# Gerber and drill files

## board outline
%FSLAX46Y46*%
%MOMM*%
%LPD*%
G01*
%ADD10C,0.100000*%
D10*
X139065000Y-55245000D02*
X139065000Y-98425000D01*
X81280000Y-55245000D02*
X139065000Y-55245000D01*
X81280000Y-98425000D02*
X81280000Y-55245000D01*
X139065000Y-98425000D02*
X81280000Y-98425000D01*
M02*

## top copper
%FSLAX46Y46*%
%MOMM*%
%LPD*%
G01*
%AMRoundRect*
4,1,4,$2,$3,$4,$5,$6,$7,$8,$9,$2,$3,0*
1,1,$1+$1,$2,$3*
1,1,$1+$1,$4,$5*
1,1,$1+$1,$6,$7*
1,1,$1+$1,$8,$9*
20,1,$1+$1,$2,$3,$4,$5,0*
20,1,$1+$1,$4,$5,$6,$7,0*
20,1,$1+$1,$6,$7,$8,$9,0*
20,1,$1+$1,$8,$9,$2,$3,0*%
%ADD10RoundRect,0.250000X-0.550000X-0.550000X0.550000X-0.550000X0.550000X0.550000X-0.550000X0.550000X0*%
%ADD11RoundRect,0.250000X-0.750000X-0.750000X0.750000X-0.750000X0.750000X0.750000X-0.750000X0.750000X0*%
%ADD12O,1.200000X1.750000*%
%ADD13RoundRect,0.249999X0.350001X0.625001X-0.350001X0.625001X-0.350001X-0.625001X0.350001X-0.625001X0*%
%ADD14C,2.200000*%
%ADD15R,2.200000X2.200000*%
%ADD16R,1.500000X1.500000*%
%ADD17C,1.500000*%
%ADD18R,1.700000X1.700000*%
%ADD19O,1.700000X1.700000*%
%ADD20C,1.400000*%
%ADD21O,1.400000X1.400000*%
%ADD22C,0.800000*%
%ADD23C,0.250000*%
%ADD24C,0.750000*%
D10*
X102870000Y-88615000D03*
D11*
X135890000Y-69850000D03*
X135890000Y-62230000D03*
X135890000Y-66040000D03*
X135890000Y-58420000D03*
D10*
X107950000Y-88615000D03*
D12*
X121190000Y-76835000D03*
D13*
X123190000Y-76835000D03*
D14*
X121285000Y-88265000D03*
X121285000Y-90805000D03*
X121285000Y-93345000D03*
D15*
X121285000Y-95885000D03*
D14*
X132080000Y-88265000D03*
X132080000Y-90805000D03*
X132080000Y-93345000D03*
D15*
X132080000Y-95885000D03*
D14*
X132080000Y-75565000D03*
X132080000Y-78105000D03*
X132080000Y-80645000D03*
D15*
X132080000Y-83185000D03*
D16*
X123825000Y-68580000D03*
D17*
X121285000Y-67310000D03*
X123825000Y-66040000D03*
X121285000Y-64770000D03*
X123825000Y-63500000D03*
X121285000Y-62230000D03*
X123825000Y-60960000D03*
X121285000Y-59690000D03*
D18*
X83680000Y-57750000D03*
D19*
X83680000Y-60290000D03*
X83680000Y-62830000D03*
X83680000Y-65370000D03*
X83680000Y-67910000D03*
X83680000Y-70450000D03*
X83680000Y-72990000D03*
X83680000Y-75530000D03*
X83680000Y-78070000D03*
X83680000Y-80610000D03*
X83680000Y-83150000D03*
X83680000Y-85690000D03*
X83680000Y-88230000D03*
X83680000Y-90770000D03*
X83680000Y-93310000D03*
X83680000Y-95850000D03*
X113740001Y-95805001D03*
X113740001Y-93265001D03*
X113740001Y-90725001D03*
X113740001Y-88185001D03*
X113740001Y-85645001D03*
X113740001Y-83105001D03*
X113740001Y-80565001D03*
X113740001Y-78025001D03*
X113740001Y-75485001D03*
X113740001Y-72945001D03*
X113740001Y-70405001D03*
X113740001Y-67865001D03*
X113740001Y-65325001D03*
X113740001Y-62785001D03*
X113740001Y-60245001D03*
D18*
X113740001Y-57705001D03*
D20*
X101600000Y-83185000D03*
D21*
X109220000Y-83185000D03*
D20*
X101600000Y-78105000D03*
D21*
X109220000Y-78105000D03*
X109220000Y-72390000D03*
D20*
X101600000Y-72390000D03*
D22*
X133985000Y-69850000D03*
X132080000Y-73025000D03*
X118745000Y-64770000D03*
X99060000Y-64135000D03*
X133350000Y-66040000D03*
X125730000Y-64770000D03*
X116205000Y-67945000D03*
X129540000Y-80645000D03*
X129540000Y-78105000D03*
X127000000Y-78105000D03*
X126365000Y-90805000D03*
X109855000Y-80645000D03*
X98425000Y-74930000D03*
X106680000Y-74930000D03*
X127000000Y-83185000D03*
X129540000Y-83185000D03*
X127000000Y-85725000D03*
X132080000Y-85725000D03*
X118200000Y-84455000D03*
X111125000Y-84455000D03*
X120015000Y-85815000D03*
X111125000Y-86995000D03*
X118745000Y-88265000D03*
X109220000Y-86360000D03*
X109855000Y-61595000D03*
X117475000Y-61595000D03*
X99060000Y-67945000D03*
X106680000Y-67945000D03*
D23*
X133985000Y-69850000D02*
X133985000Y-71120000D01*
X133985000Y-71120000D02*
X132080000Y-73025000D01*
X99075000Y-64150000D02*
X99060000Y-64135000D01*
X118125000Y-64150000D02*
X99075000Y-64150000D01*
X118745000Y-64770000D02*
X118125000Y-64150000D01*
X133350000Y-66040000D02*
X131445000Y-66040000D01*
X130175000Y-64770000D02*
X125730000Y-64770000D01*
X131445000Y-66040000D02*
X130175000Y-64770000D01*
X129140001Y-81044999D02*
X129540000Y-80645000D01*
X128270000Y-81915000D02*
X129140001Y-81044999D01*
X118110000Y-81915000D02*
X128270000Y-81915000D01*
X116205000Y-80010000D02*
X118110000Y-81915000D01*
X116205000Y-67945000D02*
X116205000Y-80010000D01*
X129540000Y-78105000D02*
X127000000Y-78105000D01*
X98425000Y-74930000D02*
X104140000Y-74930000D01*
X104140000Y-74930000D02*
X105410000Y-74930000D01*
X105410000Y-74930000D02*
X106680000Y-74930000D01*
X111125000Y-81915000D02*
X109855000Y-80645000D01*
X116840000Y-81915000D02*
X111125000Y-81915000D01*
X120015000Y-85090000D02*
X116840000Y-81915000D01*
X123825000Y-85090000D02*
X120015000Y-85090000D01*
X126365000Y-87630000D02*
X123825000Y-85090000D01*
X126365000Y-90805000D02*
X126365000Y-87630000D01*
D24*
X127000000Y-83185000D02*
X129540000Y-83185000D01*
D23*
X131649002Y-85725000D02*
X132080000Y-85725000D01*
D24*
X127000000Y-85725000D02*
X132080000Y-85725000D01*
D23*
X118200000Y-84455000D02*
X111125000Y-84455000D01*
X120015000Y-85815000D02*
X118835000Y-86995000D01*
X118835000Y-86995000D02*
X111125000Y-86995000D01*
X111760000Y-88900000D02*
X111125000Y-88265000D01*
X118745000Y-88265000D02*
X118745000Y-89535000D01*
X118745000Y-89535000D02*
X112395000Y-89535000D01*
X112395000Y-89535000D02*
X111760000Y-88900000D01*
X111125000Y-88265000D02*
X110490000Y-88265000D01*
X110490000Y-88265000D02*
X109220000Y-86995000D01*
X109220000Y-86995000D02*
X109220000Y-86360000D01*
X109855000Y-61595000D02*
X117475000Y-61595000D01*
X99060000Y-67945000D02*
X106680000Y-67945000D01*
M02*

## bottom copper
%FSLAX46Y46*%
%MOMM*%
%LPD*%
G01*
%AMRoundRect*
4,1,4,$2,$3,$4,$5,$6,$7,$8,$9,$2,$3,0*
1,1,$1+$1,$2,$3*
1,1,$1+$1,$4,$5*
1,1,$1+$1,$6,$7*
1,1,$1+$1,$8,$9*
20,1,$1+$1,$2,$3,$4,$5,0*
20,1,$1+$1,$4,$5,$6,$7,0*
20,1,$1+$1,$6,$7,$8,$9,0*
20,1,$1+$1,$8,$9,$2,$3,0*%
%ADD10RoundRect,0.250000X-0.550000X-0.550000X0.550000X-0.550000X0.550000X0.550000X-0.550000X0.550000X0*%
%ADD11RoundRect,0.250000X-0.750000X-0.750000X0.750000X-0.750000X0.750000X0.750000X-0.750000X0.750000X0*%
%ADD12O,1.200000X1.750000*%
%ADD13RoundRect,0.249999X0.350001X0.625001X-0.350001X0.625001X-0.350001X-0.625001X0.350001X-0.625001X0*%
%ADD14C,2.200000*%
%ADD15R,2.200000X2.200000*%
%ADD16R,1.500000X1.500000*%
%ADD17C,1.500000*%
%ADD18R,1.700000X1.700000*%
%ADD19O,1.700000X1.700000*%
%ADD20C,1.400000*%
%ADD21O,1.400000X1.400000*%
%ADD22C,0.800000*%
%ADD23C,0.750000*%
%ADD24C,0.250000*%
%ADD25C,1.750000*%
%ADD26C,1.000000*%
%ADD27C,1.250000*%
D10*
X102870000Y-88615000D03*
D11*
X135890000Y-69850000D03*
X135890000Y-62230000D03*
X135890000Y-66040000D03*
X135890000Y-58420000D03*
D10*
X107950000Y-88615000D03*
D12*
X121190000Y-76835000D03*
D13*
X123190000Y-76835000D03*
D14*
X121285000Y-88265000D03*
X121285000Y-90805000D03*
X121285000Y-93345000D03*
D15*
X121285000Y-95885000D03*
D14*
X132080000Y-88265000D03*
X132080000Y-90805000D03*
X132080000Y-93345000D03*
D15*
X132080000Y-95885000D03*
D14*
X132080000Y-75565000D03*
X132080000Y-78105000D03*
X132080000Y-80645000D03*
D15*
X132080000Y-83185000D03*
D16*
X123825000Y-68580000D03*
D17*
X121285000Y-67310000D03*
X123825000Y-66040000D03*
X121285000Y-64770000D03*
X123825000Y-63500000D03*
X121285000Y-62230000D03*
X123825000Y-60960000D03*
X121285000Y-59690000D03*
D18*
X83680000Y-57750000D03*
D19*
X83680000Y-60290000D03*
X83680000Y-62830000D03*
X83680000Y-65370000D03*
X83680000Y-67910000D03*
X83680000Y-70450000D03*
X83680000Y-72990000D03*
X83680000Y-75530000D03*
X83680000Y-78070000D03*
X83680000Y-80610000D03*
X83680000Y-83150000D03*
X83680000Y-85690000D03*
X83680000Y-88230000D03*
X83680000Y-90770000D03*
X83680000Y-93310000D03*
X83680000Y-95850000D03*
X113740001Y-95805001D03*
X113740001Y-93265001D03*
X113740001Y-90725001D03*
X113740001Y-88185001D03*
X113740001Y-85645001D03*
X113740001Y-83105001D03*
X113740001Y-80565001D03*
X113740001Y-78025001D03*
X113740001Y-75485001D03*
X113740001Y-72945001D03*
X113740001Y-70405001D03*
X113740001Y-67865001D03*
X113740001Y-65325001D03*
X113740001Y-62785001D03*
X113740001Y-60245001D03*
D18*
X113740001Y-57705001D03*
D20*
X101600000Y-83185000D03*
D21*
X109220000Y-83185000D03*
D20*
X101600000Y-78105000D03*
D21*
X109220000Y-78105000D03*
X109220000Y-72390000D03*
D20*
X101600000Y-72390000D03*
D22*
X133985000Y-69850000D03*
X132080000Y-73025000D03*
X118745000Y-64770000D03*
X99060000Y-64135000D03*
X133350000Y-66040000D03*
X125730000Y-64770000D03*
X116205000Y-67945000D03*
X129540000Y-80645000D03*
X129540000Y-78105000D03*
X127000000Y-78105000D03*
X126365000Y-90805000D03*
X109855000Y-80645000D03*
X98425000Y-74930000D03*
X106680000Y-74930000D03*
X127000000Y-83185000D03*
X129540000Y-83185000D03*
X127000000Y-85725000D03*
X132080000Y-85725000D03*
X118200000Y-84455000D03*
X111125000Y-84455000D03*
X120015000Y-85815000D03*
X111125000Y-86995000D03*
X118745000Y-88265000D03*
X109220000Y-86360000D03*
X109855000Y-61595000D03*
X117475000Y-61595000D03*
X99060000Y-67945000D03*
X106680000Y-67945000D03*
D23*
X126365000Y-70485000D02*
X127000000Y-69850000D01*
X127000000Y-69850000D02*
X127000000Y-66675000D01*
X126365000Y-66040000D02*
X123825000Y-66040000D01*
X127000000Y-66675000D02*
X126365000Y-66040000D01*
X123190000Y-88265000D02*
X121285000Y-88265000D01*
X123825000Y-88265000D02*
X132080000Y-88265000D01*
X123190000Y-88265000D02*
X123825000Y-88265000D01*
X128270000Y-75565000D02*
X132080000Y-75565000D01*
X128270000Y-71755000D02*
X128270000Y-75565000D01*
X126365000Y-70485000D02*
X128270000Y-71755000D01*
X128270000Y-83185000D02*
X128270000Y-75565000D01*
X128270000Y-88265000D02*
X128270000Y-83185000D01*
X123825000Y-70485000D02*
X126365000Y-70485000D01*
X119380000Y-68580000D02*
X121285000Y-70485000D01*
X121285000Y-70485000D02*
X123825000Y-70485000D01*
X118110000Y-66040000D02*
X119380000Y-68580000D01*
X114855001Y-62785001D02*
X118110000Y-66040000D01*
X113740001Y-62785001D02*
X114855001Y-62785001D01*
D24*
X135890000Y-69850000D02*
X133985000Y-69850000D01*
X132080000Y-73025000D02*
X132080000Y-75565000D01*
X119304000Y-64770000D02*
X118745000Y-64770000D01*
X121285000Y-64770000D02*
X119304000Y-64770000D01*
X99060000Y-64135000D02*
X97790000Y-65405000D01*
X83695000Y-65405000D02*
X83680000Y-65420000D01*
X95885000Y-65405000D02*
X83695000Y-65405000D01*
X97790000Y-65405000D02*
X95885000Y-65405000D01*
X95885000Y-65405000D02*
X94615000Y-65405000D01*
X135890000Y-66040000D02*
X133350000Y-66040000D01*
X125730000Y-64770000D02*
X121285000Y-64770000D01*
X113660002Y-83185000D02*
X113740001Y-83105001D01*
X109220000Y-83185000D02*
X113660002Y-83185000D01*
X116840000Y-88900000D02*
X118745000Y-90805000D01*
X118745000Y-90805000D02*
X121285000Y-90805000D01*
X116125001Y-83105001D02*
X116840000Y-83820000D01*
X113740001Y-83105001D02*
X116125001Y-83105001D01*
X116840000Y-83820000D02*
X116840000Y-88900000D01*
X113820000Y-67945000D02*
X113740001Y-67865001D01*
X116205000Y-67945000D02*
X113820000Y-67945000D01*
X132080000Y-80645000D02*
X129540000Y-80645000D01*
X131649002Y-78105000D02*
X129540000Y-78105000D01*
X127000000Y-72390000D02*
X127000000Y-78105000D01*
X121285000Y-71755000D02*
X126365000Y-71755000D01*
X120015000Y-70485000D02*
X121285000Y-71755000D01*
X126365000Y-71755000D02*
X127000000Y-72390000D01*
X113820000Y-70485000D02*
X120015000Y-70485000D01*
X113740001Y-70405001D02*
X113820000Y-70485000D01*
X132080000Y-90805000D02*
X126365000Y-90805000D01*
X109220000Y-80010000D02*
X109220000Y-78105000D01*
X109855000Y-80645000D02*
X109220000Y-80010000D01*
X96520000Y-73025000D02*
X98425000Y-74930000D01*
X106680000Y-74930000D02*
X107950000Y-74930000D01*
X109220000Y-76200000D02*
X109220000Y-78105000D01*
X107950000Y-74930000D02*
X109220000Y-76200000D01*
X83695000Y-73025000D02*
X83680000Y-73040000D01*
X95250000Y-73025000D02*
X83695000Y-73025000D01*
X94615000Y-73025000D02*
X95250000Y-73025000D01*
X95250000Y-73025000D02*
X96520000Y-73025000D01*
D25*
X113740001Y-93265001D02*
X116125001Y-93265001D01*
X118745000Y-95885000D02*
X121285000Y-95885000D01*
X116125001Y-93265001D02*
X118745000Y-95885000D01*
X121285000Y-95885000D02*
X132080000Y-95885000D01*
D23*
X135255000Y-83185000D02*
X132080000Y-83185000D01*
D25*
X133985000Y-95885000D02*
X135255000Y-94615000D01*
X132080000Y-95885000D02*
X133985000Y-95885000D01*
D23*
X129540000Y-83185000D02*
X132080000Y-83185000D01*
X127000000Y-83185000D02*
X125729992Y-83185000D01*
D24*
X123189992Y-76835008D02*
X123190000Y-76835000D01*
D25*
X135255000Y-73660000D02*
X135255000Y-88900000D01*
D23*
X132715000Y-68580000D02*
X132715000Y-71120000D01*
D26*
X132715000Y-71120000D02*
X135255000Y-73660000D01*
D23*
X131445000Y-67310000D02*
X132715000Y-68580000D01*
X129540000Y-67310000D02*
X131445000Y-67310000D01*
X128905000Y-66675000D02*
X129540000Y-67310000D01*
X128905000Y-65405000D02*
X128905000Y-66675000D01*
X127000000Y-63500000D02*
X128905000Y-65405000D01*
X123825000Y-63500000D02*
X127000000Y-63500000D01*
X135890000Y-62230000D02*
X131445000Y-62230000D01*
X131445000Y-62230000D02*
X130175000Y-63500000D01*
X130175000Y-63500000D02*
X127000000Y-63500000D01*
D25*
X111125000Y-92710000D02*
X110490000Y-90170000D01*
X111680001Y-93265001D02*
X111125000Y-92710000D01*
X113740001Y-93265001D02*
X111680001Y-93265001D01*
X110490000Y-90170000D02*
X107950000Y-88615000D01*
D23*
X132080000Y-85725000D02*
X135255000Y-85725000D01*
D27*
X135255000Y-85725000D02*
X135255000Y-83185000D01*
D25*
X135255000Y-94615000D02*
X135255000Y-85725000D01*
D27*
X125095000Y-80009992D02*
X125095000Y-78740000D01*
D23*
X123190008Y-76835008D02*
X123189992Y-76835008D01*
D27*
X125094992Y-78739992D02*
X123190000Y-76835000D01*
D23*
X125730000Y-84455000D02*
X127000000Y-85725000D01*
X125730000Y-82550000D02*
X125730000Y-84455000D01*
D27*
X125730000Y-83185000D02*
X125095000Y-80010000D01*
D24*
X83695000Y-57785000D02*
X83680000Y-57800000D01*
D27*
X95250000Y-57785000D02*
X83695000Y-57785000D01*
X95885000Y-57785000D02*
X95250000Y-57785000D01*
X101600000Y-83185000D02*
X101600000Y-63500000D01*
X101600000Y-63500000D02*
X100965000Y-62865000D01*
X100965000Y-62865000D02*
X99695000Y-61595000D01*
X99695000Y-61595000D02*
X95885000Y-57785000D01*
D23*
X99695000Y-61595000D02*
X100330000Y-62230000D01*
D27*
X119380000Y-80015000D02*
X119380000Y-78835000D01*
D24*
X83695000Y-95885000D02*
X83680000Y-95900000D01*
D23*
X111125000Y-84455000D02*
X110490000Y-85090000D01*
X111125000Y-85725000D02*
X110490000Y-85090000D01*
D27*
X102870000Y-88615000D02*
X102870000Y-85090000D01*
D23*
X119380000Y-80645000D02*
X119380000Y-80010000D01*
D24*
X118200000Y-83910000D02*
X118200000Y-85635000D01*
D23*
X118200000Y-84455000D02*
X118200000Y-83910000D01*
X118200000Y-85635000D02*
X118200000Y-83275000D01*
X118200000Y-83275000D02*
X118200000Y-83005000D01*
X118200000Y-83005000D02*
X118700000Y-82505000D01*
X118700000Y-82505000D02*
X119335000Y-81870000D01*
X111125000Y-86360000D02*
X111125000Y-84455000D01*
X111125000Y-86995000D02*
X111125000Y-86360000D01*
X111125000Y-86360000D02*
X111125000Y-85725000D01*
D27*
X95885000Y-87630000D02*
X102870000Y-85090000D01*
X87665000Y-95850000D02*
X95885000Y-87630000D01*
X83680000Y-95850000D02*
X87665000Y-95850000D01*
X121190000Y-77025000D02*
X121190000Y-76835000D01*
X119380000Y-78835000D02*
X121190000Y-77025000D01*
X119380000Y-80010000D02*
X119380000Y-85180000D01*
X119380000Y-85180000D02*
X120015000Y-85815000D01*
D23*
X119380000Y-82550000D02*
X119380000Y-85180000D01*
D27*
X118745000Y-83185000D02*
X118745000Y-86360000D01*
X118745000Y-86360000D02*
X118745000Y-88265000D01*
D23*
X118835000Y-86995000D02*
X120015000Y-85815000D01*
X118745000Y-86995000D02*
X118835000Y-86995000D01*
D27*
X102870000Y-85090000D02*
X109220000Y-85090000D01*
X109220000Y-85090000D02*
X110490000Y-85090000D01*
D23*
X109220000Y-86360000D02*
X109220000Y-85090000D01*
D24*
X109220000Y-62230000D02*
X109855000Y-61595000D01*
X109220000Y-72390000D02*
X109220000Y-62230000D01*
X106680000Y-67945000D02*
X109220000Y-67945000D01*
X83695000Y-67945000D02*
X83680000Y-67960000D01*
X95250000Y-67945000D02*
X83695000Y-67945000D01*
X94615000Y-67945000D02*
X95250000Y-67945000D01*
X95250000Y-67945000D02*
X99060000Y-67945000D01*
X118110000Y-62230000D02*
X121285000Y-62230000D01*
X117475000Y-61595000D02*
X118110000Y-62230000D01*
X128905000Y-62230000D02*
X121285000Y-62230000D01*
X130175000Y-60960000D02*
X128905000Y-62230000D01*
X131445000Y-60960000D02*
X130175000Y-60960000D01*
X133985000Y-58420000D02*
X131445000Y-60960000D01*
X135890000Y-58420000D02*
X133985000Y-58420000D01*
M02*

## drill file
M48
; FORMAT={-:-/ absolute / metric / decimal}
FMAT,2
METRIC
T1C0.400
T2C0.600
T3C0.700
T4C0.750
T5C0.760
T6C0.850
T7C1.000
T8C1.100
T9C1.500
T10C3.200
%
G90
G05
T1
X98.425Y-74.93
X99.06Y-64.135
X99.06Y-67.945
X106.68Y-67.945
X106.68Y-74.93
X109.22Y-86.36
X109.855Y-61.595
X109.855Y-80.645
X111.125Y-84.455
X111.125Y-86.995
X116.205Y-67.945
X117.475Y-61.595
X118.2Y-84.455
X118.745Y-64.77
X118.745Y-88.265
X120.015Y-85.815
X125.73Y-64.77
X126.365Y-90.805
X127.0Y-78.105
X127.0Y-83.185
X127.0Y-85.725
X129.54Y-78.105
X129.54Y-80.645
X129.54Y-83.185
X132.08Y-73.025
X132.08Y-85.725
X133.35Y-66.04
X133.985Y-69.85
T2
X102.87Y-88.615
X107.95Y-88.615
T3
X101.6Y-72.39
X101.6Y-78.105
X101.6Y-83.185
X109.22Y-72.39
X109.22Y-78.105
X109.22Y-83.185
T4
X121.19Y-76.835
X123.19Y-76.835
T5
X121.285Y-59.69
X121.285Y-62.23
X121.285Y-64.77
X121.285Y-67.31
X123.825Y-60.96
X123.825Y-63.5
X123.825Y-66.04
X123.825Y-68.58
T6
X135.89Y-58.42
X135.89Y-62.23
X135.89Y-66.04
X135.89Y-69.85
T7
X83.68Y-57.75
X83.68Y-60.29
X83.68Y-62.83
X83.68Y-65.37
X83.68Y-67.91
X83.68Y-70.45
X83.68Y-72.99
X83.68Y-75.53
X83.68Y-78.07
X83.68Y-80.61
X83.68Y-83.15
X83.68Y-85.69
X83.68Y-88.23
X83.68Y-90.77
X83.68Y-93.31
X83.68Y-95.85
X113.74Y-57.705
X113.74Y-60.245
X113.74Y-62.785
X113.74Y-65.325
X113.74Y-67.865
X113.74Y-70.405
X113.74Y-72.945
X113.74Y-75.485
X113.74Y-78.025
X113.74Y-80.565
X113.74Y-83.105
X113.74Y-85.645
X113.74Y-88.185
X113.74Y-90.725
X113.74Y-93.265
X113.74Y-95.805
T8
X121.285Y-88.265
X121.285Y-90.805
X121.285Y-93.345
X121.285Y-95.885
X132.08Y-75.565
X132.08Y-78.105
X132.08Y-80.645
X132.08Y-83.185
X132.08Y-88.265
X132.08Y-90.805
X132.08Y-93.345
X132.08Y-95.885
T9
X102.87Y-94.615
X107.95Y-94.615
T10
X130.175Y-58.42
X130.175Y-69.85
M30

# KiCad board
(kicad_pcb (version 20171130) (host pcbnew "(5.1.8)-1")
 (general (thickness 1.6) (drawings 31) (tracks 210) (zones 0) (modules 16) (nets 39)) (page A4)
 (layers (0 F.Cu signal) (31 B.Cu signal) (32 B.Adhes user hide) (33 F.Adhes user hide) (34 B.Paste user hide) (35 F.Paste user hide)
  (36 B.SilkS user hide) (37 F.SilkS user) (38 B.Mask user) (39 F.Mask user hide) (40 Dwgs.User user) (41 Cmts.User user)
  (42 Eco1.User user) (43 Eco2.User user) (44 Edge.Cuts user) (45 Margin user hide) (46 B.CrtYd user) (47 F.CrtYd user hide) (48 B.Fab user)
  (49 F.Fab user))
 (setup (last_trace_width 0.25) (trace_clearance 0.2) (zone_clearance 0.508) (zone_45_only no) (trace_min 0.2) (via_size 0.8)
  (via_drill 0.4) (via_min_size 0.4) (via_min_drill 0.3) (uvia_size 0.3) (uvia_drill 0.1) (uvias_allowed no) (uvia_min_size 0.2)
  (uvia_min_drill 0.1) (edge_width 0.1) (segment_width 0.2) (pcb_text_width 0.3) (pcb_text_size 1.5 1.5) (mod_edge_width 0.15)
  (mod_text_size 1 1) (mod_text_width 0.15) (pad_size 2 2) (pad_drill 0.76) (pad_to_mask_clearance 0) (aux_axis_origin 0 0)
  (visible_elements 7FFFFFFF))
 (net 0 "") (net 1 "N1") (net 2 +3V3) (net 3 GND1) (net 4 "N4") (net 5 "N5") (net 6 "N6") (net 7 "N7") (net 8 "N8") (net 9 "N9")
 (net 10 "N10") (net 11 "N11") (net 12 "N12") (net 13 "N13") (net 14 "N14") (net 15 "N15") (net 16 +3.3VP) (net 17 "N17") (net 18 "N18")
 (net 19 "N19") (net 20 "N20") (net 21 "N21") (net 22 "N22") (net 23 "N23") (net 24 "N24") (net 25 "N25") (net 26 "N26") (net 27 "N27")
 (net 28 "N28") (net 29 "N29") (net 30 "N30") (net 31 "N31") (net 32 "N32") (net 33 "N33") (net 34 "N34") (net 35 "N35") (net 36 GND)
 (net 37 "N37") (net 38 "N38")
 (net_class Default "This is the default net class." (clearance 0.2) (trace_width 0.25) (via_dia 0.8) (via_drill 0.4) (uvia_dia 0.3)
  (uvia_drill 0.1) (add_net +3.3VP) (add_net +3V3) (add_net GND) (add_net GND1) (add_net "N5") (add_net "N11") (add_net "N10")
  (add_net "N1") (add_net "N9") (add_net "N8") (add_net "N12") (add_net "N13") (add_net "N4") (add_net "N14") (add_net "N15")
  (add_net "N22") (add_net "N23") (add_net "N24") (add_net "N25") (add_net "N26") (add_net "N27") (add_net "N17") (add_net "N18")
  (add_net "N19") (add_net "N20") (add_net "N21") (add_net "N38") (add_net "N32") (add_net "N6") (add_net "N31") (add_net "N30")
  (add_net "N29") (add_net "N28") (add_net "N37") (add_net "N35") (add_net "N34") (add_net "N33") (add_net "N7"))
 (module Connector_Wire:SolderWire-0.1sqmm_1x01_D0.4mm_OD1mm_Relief (layer F.Cu) (at 102.87 88.615)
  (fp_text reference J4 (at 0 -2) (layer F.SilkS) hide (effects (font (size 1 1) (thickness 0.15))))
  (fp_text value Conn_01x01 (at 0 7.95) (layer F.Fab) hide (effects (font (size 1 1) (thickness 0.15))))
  (pad "" np_thru_hole circle (at 0 6) (size 1.5 1.5) (drill 1.5) (layers *.Cu *.Mask))
  (pad 1 thru_hole roundrect (at 0 0) (size 1.6 1.6) (drill 0.6) (layers *.Cu *.Mask) (roundrect_rratio 0.15625) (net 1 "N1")))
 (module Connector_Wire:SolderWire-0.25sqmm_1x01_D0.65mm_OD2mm (layer F.Cu) (at 135.89 69.85)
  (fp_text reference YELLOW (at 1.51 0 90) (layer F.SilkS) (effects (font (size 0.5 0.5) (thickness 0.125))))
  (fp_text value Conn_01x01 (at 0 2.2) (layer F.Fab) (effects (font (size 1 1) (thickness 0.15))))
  (pad 1 thru_hole roundrect (at 0 0) (size 2 2) (drill 0.85) (layers *.Cu *.Mask) (roundrect_rratio 0.125) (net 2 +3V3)))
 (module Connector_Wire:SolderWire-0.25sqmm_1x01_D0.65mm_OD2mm (layer F.Cu) (at 135.89 62.23)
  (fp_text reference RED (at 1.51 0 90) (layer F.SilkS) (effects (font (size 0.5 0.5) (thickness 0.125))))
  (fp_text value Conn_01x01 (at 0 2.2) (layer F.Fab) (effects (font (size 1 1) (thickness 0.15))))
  (pad 1 thru_hole roundrect (at 0 0) (size 2 2) (drill 0.85) (layers *.Cu *.Mask) (roundrect_rratio 0.125) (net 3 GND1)))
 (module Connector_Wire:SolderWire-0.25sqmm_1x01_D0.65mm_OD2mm (layer F.Cu) (at 135.89 66.04)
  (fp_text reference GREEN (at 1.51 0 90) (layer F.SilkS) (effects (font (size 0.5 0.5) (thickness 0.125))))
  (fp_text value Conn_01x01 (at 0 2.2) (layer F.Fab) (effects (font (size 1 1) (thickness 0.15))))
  (pad 1 thru_hole roundrect (at 0 0) (size 2 2) (drill 0.85) (layers *.Cu *.Mask) (roundrect_rratio 0.125) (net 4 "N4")))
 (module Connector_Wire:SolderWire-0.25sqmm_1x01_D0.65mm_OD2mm (layer F.Cu) (at 135.89 58.42)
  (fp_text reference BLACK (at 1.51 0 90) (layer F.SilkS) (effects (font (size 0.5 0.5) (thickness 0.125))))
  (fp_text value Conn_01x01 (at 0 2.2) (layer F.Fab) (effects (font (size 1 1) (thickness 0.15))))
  (pad 1 thru_hole roundrect (at 0 0) (size 2 2) (drill 0.85) (layers *.Cu *.Mask) (roundrect_rratio 0.125) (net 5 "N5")))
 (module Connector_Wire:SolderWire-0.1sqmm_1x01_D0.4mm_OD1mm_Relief (layer F.Cu) (at 107.95 88.615)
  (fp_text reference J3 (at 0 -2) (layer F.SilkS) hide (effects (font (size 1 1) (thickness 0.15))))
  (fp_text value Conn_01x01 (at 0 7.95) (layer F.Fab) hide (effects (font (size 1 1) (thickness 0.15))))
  (pad "" np_thru_hole circle (at 0 6) (size 1.5 1.5) (drill 1.5) (layers *.Cu *.Mask))
  (pad 1 thru_hole roundrect (at 0 0) (size 1.6 1.6) (drill 0.6) (layers *.Cu *.Mask) (roundrect_rratio 0.15625) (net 3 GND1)))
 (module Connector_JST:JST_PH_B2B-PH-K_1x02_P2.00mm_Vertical (layer F.Cu) (at 123.19 76.835 180)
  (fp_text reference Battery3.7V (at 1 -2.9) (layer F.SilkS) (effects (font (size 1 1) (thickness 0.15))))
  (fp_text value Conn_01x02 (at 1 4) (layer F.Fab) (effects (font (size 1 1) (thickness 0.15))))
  (pad 2 thru_hole oval (at 2 0 180) (size 1.2 1.75) (drill 0.75) (layers *.Cu *.Mask) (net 1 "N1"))
  (pad 1 thru_hole roundrect (at 0 0 180) (size 1.2 1.75) (drill 0.75) (layers *.Cu *.Mask) (roundrect_rratio 0.2083325) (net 3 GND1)))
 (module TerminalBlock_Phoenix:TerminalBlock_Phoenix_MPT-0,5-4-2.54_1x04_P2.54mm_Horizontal (layer F.Cu) (at 121.285 95.885 90)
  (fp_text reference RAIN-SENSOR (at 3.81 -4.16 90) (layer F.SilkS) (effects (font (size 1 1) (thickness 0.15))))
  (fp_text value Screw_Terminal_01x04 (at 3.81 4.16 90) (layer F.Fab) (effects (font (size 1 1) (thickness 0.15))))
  (pad 4 thru_hole circle (at 7.62 0 90) (size 2.2 2.2) (drill 1.1) (layers *.Cu *.Mask) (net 2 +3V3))
  (pad 3 thru_hole circle (at 5.08 0 90) (size 2.2 2.2) (drill 1.1) (layers *.Cu *.Mask) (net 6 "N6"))
  (pad 2 thru_hole circle (at 2.54 0 90) (size 2.2 2.2) (drill 1.1) (layers *.Cu *.Mask) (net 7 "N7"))
  (pad 1 thru_hole rect (at 0 0 90) (size 2.2 2.2) (drill 1.1) (layers *.Cu *.Mask) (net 3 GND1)))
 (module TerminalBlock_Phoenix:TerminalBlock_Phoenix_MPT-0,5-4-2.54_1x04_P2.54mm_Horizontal (layer F.Cu) (at 132.08 95.885 90)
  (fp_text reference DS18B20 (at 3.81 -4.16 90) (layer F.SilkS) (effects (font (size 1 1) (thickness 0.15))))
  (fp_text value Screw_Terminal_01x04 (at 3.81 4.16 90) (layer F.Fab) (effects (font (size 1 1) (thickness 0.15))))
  (pad 4 thru_hole circle (at 7.62 0 90) (size 2.2 2.2) (drill 1.1) (layers *.Cu *.Mask) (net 2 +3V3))
  (pad 3 thru_hole circle (at 5.08 0 90) (size 2.2 2.2) (drill 1.1) (layers *.Cu *.Mask) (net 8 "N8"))
  (pad 2 thru_hole circle (at 2.54 0 90) (size 2.2 2.2) (drill 1.1) (layers *.Cu *.Mask) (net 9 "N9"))
  (pad 1 thru_hole rect (at 0 0 90) (size 2.2 2.2) (drill 1.1) (layers *.Cu *.Mask) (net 3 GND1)))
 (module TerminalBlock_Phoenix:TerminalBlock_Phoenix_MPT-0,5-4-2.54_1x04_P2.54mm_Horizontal (layer F.Cu) (at 132.08 83.185 90)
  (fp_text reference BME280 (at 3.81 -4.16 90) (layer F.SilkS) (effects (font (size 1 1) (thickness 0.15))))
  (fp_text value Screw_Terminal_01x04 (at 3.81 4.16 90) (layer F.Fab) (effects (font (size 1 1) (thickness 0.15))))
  (pad 4 thru_hole circle (at 7.62 0 90) (size 2.2 2.2) (drill 1.1) (layers *.Cu *.Mask) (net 2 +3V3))
  (pad 3 thru_hole circle (at 5.08 0 90) (size 2.2 2.2) (drill 1.1) (layers *.Cu *.Mask) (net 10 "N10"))
  (pad 2 thru_hole circle (at 2.54 0 90) (size 2.2 2.2) (drill 1.1) (layers *.Cu *.Mask) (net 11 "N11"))
  (pad 1 thru_hole rect (at 0 0 90) (size 2.2 2.2) (drill 1.1) (layers *.Cu *.Mask) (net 3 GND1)))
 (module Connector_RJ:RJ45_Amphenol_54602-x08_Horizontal (layer F.Cu) (at 123.825 68.58 90)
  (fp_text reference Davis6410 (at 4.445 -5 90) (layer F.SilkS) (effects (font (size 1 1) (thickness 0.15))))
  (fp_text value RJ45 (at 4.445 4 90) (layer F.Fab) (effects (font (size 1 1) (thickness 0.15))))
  (pad "" np_thru_hole circle (at 10.16 6.35 90) (size 3.2 3.2) (drill 3.2) (layers *.Cu *.Mask))
  (pad "" np_thru_hole circle (at -1.27 6.35 90) (size 3.2 3.2) (drill 3.2) (layers *.Cu *.Mask))
  (pad 1 thru_hole rect (at 0 0 90) (size 1.5 1.5) (drill 0.76) (layers *.Cu *.Mask) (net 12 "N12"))
  (pad 2 thru_hole circle (at 1.27 -2.54 90) (size 1.5 1.5) (drill 0.76) (layers *.Cu *.Mask) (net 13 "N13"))
  (pad 3 thru_hole circle (at 2.54 0 90) (size 1.5 1.5) (drill 0.76) (layers *.Cu *.Mask) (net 2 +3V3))
  (pad 4 thru_hole circle (at 3.81 -2.54 90) (size 1.5 1.5) (drill 0.76) (layers *.Cu *.Mask) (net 4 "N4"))
  (pad 5 thru_hole circle (at 5.08 0 90) (size 1.5 1.5) (drill 0.76) (layers *.Cu *.Mask) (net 3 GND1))
  (pad 6 thru_hole circle (at 6.35 -2.54 90) (size 1.5 1.5) (drill 0.76) (layers *.Cu *.Mask) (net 5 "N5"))
  (pad 7 thru_hole circle (at 7.62 0 90) (size 1.5 1.5) (drill 0.76) (layers *.Cu *.Mask) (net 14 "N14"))
  (pad 8 thru_hole circle (at 8.89 -2.54 90) (size 1.5 1.5) (drill 0.76) (layers *.Cu *.Mask) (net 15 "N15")))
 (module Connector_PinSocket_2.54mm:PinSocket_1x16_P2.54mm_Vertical (layer F.Cu) (at 83.68 57.75)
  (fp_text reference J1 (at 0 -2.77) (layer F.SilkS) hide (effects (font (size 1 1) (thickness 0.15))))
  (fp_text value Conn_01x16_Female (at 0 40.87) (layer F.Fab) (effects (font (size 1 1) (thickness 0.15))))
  (pad 1 thru_hole rect (at 0 0) (size 1.7 1.7) (drill 1) (layers *.Cu *.Mask) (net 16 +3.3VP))
  (pad 2 thru_hole oval (at 0 2.54) (size 1.7 1.7) (drill 1) (layers *.Cu *.Mask) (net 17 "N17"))
  (pad 3 thru_hole oval (at 0 5.08) (size 1.7 1.7) (drill 1) (layers *.Cu *.Mask) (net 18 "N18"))
  (pad 4 thru_hole oval (at 0 7.62) (size 1.7 1.7) (drill 1) (layers *.Cu *.Mask) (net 4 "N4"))
  (pad 5 thru_hole oval (at 0 10.16) (size 1.7 1.7) (drill 1) (layers *.Cu *.Mask) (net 5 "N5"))
  (pad 6 thru_hole oval (at 0 12.7) (size 1.7 1.7) (drill 1) (layers *.Cu *.Mask) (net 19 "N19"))
  (pad 7 thru_hole oval (at 0 15.24) (size 1.7 1.7) (drill 1) (layers *.Cu *.Mask) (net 8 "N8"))
  (pad 8 thru_hole oval (at 0 17.78) (size 1.7 1.7) (drill 1) (layers *.Cu *.Mask) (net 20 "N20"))
  (pad 9 thru_hole oval (at 0 20.32) (size 1.7 1.7) (drill 1) (layers *.Cu *.Mask) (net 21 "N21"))
  (pad 10 thru_hole oval (at 0 22.86) (size 1.7 1.7) (drill 1) (layers *.Cu *.Mask) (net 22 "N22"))
  (pad 11 thru_hole oval (at 0 25.4) (size 1.7 1.7) (drill 1) (layers *.Cu *.Mask) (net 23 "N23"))
  (pad 12 thru_hole oval (at 0 27.94) (size 1.7 1.7) (drill 1) (layers *.Cu *.Mask) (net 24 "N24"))
  (pad 13 thru_hole oval (at 0 30.48) (size 1.7 1.7) (drill 1) (layers *.Cu *.Mask) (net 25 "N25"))
  (pad 14 thru_hole oval (at 0 33.02) (size 1.7 1.7) (drill 1) (layers *.Cu *.Mask) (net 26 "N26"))
  (pad 15 thru_hole oval (at 0 35.56) (size 1.7 1.7) (drill 1) (layers *.Cu *.Mask) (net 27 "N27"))
  (pad 16 thru_hole oval (at 0 38.1) (size 1.7 1.7) (drill 1) (layers *.Cu *.Mask) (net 1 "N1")))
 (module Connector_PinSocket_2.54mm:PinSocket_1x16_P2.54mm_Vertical (layer F.Cu) (at 113.740001 57.705001)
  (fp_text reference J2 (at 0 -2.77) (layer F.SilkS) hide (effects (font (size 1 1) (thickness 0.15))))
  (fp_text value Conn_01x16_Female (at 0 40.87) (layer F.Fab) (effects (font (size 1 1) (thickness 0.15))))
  (pad 16 thru_hole oval (at 0 38.1) (size 1.7 1.7) (drill 1) (layers *.Cu *.Mask) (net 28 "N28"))
  (pad 15 thru_hole oval (at 0 35.56) (size 1.7 1.7) (drill 1) (layers *.Cu *.Mask) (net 3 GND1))
  (pad 14 thru_hole oval (at 0 33.02) (size 1.7 1.7) (drill 1) (layers *.Cu *.Mask) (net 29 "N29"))
  (pad 13 thru_hole oval (at 0 30.48) (size 1.7 1.7) (drill 1) (layers *.Cu *.Mask) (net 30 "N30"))
  (pad 12 thru_hole oval (at 0 27.94) (size 1.7 1.7) (drill 1) (layers *.Cu *.Mask) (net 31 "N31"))
  (pad 11 thru_hole oval (at 0 25.4) (size 1.7 1.7) (drill 1) (layers *.Cu *.Mask) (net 6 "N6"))
  (pad 10 thru_hole oval (at 0 22.86) (size 1.7 1.7) (drill 1) (layers *.Cu *.Mask) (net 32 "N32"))
  (pad 9 thru_hole oval (at 0 20.32) (size 1.7 1.7) (drill 1) (layers *.Cu *.Mask) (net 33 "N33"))
  (pad 8 thru_hole oval (at 0 17.78) (size 1.7 1.7) (drill 1) (layers *.Cu *.Mask) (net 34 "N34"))
  (pad 7 thru_hole oval (at 0 15.24) (size 1.7 1.7) (drill 1) (layers *.Cu *.Mask) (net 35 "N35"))
  (pad 6 thru_hole oval (at 0 12.7) (size 1.7 1.7) (drill 1) (layers *.Cu *.Mask) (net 10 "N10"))
  (pad 5 thru_hole oval (at 0 10.16) (size 1.7 1.7) (drill 1) (layers *.Cu *.Mask) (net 11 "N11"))
  (pad 4 thru_hole oval (at 0 7.62) (size 1.7 1.7) (drill 1) (layers *.Cu *.Mask) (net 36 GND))
  (pad 3 thru_hole oval (at 0 5.08) (size 1.7 1.7) (drill 1) (layers *.Cu *.Mask) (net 2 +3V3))
  (pad 2 thru_hole oval (at 0 2.54) (size 1.7 1.7) (drill 1) (layers *.Cu *.Mask) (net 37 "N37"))
  (pad 1 thru_hole rect (at 0 0) (size 1.7 1.7) (drill 1) (layers *.Cu *.Mask) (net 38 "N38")))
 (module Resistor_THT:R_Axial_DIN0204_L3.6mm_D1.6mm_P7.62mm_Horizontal (layer F.Cu) (at 101.6 83.185)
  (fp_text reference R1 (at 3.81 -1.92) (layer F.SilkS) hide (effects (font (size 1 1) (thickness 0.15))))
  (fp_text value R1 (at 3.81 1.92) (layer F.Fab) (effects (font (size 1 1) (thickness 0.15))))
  (pad 1 thru_hole circle (at 0 0) (size 1.4 1.4) (drill 0.7) (layers *.Cu *.Mask) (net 16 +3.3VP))
  (pad 2 thru_hole oval (at 7.62 0) (size 1.4 1.4) (drill 0.7) (layers *.Cu *.Mask) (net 6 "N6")))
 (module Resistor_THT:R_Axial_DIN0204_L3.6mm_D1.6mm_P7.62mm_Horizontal (layer F.Cu) (at 101.6 78.105)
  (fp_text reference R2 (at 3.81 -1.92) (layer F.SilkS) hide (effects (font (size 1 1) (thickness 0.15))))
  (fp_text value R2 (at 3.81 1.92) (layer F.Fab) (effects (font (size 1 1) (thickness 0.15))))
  (pad 1 thru_hole circle (at 0 0) (size 1.4 1.4) (drill 0.7) (layers *.Cu *.Mask) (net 16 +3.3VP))
  (pad 2 thru_hole oval (at 7.62 0) (size 1.4 1.4) (drill 0.7) (layers *.Cu *.Mask) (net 8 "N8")))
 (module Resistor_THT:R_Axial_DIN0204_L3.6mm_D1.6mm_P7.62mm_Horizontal (layer F.Cu) (at 101.6 72.39)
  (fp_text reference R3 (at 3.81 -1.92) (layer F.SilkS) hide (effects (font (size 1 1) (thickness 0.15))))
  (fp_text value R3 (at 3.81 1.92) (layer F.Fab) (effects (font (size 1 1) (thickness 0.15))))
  (pad 2 thru_hole oval (at 7.62 0) (size 1.4 1.4) (drill 0.7) (layers *.Cu *.Mask) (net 5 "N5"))
  (pad 1 thru_hole circle (at 0 0) (size 1.4 1.4) (drill 0.7) (layers *.Cu *.Mask) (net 16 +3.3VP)))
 (gr_line (start 139.065 55.245) (end 139.065 98.425) (layer Edge.Cuts) (width 0.1))
 (gr_line (start 81.28 55.245) (end 139.065 55.245) (layer Edge.Cuts) (width 0.1))
 (gr_line (start 81.28 98.425) (end 81.28 55.245) (layer Edge.Cuts) (width 0.1))
 (gr_line (start 139.065 98.425) (end 81.28 98.425) (layer Edge.Cuts) (width 0.1))
 (segment (start 126.365 70.485) (end 127 69.85) (width 0.75) (layer B.Cu) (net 2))
 (segment (start 127 69.85) (end 127 66.675) (width 0.75) (layer B.Cu) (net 2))
 (segment (start 126.365 66.04) (end 123.825 66.04) (width 0.75) (layer B.Cu) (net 2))
 (segment (start 127 66.675) (end 126.365 66.04) (width 0.75) (layer B.Cu) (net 2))
 (segment (start 123.19 88.265) (end 121.285 88.265) (width 0.75) (layer B.Cu) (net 2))
 (segment (start 123.825 88.265) (end 132.08 88.265) (width 0.75) (layer B.Cu) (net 2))
 (segment (start 123.19 88.265) (end 123.825 88.265) (width 0.75) (layer B.Cu) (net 2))
 (segment (start 128.27 75.565) (end 132.08 75.565) (width 0.75) (layer B.Cu) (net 2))
 (segment (start 128.27 71.755) (end 128.27 75.565) (width 0.75) (layer B.Cu) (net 2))
 (segment (start 126.365 70.485) (end 128.27 71.755) (width 0.75) (layer B.Cu) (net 2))
 (segment (start 128.27 83.185) (end 128.27 75.565) (width 0.75) (layer B.Cu) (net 2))
 (segment (start 128.27 88.265) (end 128.27 83.185) (width 0.75) (layer B.Cu) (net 2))
 (segment (start 123.825 70.485) (end 126.365 70.485) (width 0.75) (layer B.Cu) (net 2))
 (segment (start 119.38 68.58) (end 121.285 70.485) (width 0.75) (layer B.Cu) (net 2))
 (segment (start 121.285 70.485) (end 123.825 70.485) (width 0.75) (layer B.Cu) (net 2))
 (segment (start 118.11 66.04) (end 119.38 68.58) (width 0.75) (layer B.Cu) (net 2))
 (segment (start 114.855001 62.785001) (end 118.11 66.04) (width 0.75) (layer B.Cu) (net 2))
 (segment (start 113.740001 62.785001) (end 114.855001 62.785001) (width 0.75) (layer B.Cu) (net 2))
 (via (at 133.985 69.85) (size 0.8) (drill 0.4) (layers F.Cu B.Cu) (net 2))
 (segment (start 135.89 69.85) (end 133.985 69.85) (width 0.25) (layer B.Cu) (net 2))
 (segment (start 133.985 69.85) (end 133.985 71.12) (width 0.25) (layer F.Cu) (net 2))
 (via (at 132.08 73.025) (size 0.8) (drill 0.4) (layers F.Cu B.Cu) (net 2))
 (segment (start 133.985 71.12) (end 132.08 73.025) (width 0.25) (layer F.Cu) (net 2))
 (segment (start 132.08 73.025) (end 132.08 75.565) (width 0.25) (layer B.Cu) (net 2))
 (via (at 118.745 64.77) (size 0.8) (drill 0.4) (layers F.Cu B.Cu) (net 4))
 (segment (start 119.304 64.77) (end 118.745 64.77) (width 0.25) (layer B.Cu) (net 4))
 (segment (start 121.285 64.77) (end 119.304 64.77) (width 0.25) (layer B.Cu) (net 4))
 (via (at 99.06 64.135) (size 0.8) (drill 0.4) (layers F.Cu B.Cu) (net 4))
 (segment (start 99.075 64.15) (end 99.06 64.135) (width 0.25) (layer F.Cu) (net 4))
 (segment (start 118.125 64.15) (end 99.075 64.15) (width 0.25) (layer F.Cu) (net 4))
 (segment (start 118.745 64.77) (end 118.125 64.15) (width 0.25) (layer F.Cu) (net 4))
 (segment (start 99.06 64.135) (end 97.79 65.405) (width 0.25) (layer B.Cu) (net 4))
 (segment (start 83.695 65.405) (end 83.68 65.42) (width 0.25) (layer B.Cu) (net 4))
 (segment (start 95.885 65.405) (end 83.695 65.405) (width 0.25) (layer B.Cu) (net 4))
 (segment (start 97.79 65.405) (end 95.885 65.405) (width 0.25) (layer B.Cu) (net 4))
 (segment (start 95.885 65.405) (end 94.615 65.405) (width 0.25) (layer B.Cu) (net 4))
 (via (at 133.35 66.04) (size 0.8) (drill 0.4) (layers F.Cu B.Cu) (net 4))
 (segment (start 135.89 66.04) (end 133.35 66.04) (width 0.25) (layer B.Cu) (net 4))
 (segment (start 133.35 66.04) (end 131.445 66.04) (width 0.25) (layer F.Cu) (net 4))
 (via (at 125.73 64.77) (size 0.8) (drill 0.4) (layers F.Cu B.Cu) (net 4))
 (segment (start 130.175 64.77) (end 125.73 64.77) (width 0.25) (layer F.Cu) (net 4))
 (segment (start 131.445 66.04) (end 130.175 64.77) (width 0.25) (layer F.Cu) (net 4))
 (segment (start 125.73 64.77) (end 121.285 64.77) (width 0.25) (layer B.Cu) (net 4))
 (segment (start 113.660002 83.185) (end 113.740001 83.105001) (width 0.25) (layer B.Cu) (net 6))
 (segment (start 109.22 83.185) (end 113.660002 83.185) (width 0.25) (layer B.Cu) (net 6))
 (segment (start 116.84 88.9) (end 118.745 90.805) (width 0.25) (layer B.Cu) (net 6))
 (segment (start 118.745 90.805) (end 121.285 90.805) (width 0.25) (layer B.Cu) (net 6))
 (segment (start 116.125001 83.105001) (end 116.84 83.82) (width 0.25) (layer B.Cu) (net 6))
 (segment (start 113.740001 83.105001) (end 116.125001 83.105001) (width 0.25) (layer B.Cu) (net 6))
 (segment (start 116.84 83.82) (end 116.84 88.9) (width 0.25) (layer B.Cu) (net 6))
 (via (at 116.205 67.945) (size 0.8) (drill 0.4) (layers F.Cu B.Cu) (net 11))
 (segment (start 113.82 67.945) (end 113.740001 67.865001) (width 0.25) (layer B.Cu) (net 11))
 (segment (start 116.205 67.945) (end 113.82 67.945) (width 0.25) (layer B.Cu) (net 11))
 (segment (start 132.08 80.645) (end 129.54 80.645) (width 0.25) (layer B.Cu) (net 11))
 (via (at 129.54 80.645) (size 0.8) (drill 0.4) (layers F.Cu B.Cu) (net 11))
 (segment (start 129.140001 81.044999) (end 129.54 80.645) (width 0.25) (layer F.Cu) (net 11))
 (segment (start 128.27 81.915) (end 129.140001 81.044999) (width 0.25) (layer F.Cu) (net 11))
 (segment (start 118.11 81.915) (end 128.27 81.915) (width 0.25) (layer F.Cu) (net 11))
 (segment (start 116.205 80.01) (end 118.11 81.915) (width 0.25) (layer F.Cu) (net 11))
 (segment (start 116.205 67.945) (end 116.205 80.01) (width 0.25) (layer F.Cu) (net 11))
 (segment (start 131.649002 78.105) (end 129.54 78.105) (width 0.25) (layer B.Cu) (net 10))
 (via (at 129.54 78.105) (size 0.8) (drill 0.4) (layers F.Cu B.Cu) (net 10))
 (segment (start 129.54 78.105) (end 127 78.105) (width 0.25) (layer F.Cu) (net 10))
 (via (at 127 78.105) (size 0.8) (drill 0.4) (layers F.Cu B.Cu) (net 10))
 (segment (start 127 72.39) (end 127 78.105) (width 0.25) (layer B.Cu) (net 10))
 (segment (start 121.285 71.755) (end 126.365 71.755) (width 0.25) (layer B.Cu) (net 10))
 (segment (start 120.015 70.485) (end 121.285 71.755) (width 0.25) (layer B.Cu) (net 10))
 (segment (start 126.365 71.755) (end 127 72.39) (width 0.25) (layer B.Cu) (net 10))
 (segment (start 113.82 70.485) (end 120.015 70.485) (width 0.25) (layer B.Cu) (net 10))
 (segment (start 113.740001 70.405001) (end 113.82 70.485) (width 0.25) (layer B.Cu) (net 10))
 (via (at 126.365 90.805) (size 0.8) (drill 0.4) (layers F.Cu B.Cu) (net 8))
 (segment (start 132.08 90.805) (end 126.365 90.805) (width 0.25) (layer B.Cu) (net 8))
 (via (at 109.855 80.645) (size 0.8) (drill 0.4) (layers F.Cu B.Cu) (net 8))
 (segment (start 109.22 80.01) (end 109.22 78.105) (width 0.25) (layer B.Cu) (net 8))
 (segment (start 109.855 80.645) (end 109.22 80.01) (width 0.25) (layer B.Cu) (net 8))
 (via (at 98.425 74.93) (size 0.8) (drill 0.4) (layers F.Cu B.Cu) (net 8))
 (segment (start 96.52 73.025) (end 98.425 74.93) (width 0.25) (layer B.Cu) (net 8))
 (segment (start 98.425 74.93) (end 104.14 74.93) (width 0.25) (layer F.Cu) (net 8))
 (segment (start 104.14 74.93) (end 105.41 74.93) (width 0.25) (layer F.Cu) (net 8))
 (via (at 106.68 74.93) (size 0.8) (drill 0.4) (layers F.Cu B.Cu) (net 8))
 (segment (start 105.41 74.93) (end 106.68 74.93) (width 0.25) (layer F.Cu) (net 8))
 (segment (start 106.68 74.93) (end 107.95 74.93) (width 0.25) (layer B.Cu) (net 8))
 (segment (start 109.22 76.2) (end 109.22 78.105) (width 0.25) (layer B.Cu) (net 8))
 (segment (start 107.95 74.93) (end 109.22 76.2) (width 0.25) (layer B.Cu) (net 8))
 (segment (start 111.125 81.915) (end 109.855 80.645) (width 0.25) (layer F.Cu) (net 8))
 (segment (start 116.84 81.915) (end 111.125 81.915) (width 0.25) (layer F.Cu) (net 8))
 (segment (start 120.015 85.09) (end 116.84 81.915) (width 0.25) (layer F.Cu) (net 8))
 (segment (start 123.825 85.09) (end 120.015 85.09) (width 0.25) (layer F.Cu) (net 8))
 (segment (start 126.365 87.63) (end 123.825 85.09) (width 0.25) (layer F.Cu) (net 8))
 (segment (start 126.365 90.805) (end 126.365 87.63) (width 0.25) (layer F.Cu) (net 8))
 (segment (start 83.695 73.025) (end 83.68 73.04) (width 0.25) (layer B.Cu) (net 8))
 (segment (start 95.25 73.025) (end 83.695 73.025) (width 0.25) (layer B.Cu) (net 8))
 (segment (start 94.615 73.025) (end 95.25 73.025) (width 0.25) (layer B.Cu) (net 8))
 (segment (start 95.25 73.025) (end 96.52 73.025) (width 0.25) (layer B.Cu) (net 8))
 (segment (start 113.740001 93.265001) (end 116.125001 93.265001) (width 1.75) (layer B.Cu) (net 3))
 (segment (start 118.745 95.885) (end 121.285 95.885) (width 1.75) (layer B.Cu) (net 3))
 (segment (start 116.125001 93.265001) (end 118.745 95.885) (width 1.75) (layer B.Cu) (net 3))
 (segment (start 121.285 95.885) (end 132.08 95.885) (width 1.75) (layer B.Cu) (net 3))
 (segment (start 135.255 83.185) (end 132.08 83.185) (width 0.75) (layer B.Cu) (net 3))
 (segment (start 133.985 95.885) (end 135.255 94.615) (width 1.75) (layer B.Cu) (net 3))
 (segment (start 132.08 95.885) (end 133.985 95.885) (width 1.75) (layer B.Cu) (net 3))
 (via (at 127 83.185) (size 0.8) (drill 0.4) (layers F.Cu B.Cu) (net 3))
 (via (at 129.54 83.185) (size 0.8) (drill 0.4) (layers F.Cu B.Cu) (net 3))
 (segment (start 127 83.185) (end 129.54 83.185) (width 0.75) (layer F.Cu) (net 3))
 (segment (start 129.54 83.185) (end 132.08 83.185) (width 0.75) (layer B.Cu) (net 3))
 (segment (start 127 83.185) (end 125.729992 83.185) (width 0.75) (layer B.Cu) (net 3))
 (segment (start 123.189992 76.835008) (end 123.19 76.835) (width 0.25) (layer B.Cu) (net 3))
 (segment (start 135.255 73.66) (end 135.255 88.9) (width 1.75) (layer B.Cu) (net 3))
 (segment (start 132.715 68.58) (end 132.715 71.12) (width 0.75) (layer B.Cu) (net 3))
 (segment (start 132.715 71.12) (end 135.255 73.66) (width 1) (layer B.Cu) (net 3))
 (segment (start 131.445 67.31) (end 132.715 68.58) (width 0.75) (layer B.Cu) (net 3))
 (segment (start 129.54 67.31) (end 131.445 67.31) (width 0.75) (layer B.Cu) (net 3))
 (segment (start 128.905 66.675) (end 129.54 67.31) (width 0.75) (layer B.Cu) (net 3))
 (segment (start 128.905 65.405) (end 128.905 66.675) (width 0.75) (layer B.Cu) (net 3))
 (segment (start 127 63.5) (end 128.905 65.405) (width 0.75) (layer B.Cu) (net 3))
 (segment (start 123.825 63.5) (end 127 63.5) (width 0.75) (layer B.Cu) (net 3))
 (segment (start 135.89 62.23) (end 131.445 62.23) (width 0.75) (layer B.Cu) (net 3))
 (segment (start 131.445 62.23) (end 130.175 63.5) (width 0.75) (layer B.Cu) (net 3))
 (segment (start 130.175 63.5) (end 127 63.5) (width 0.75) (layer B.Cu) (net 3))
 (segment (start 111.125 92.71) (end 110.49 90.17) (width 1.75) (layer B.Cu) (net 3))
 (segment (start 111.680001 93.265001) (end 111.125 92.71) (width 1.75) (layer B.Cu) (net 3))
 (segment (start 113.740001 93.265001) (end 111.680001 93.265001) (width 1.75) (layer B.Cu) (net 3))
 (segment (start 110.49 90.17) (end 107.95 88.615) (width 1.75) (layer B.Cu) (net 3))
 (via (at 127 85.725) (size 0.8) (drill 0.4) (layers F.Cu B.Cu) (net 3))
 (via (at 132.08 85.725) (size 0.8) (drill 0.4) (layers F.Cu B.Cu) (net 3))
 (segment (start 131.649002 85.725) (end 132.08 85.725) (width 0.25) (layer F.Cu) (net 3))
 (segment (start 132.08 85.725) (end 135.255 85.725) (width 0.75) (layer B.Cu) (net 3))
 (segment (start 135.255 85.725) (end 135.255 83.185) (width 1.25) (layer B.Cu) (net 3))
 (segment (start 135.255 94.615) (end 135.255 85.725) (width 1.75) (layer B.Cu) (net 3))
 (segment (start 125.095 80.009992) (end 125.095 78.74) (width 1.25) (layer B.Cu) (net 3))
 (segment (start 123.190008 76.835008) (end 123.189992 76.835008) (width 0.75) (layer B.Cu) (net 3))
 (segment (start 127 85.725) (end 132.08 85.725) (width 0.75) (layer F.Cu) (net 3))
 (segment (start 125.094992 78.739992) (end 123.19 76.835) (width 1.25) (layer B.Cu) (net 3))
 (segment (start 125.73 84.455) (end 127 85.725) (width 0.75) (layer B.Cu) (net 3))
 (segment (start 125.73 82.55) (end 125.73 84.455) (width 0.75) (layer B.Cu) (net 3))
 (segment (start 125.73 83.185) (end 125.095 80.01) (width 1.25) (layer B.Cu) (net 3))
 (segment (start 83.695 57.785) (end 83.68 57.8) (width 0.25) (layer B.Cu) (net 16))
 (segment (start 95.25 57.785) (end 83.695 57.785) (width 1.25) (layer B.Cu) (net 16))
 (segment (start 95.885 57.785) (end 95.25 57.785) (width 1.25) (layer B.Cu) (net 16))
 (segment (start 101.6 83.185) (end 101.6 63.5) (width 1.25) (layer B.Cu) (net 16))
 (segment (start 101.6 63.5) (end 100.965 62.865) (width 1.25) (layer B.Cu) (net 16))
 (segment (start 100.965 62.865) (end 99.695 61.595) (width 1.25) (layer B.Cu) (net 16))
 (segment (start 99.695 61.595) (end 95.885 57.785) (width 1.25) (layer B.Cu) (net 16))
 (segment (start 99.695 61.595) (end 100.33 62.23) (width 0.75) (layer B.Cu) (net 16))
 (via (at 118.2 84.455) (size 0.8) (drill 0.4) (layers F.Cu B.Cu) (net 1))
 (via (at 111.125 84.455) (size 0.8) (drill 0.4) (layers F.Cu B.Cu) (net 1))
 (segment (start 118.2 84.455) (end 111.125 84.455) (width 0.25) (layer F.Cu) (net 1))
 (segment (start 119.38 80.015) (end 119.38 78.835) (width 1.25) (layer B.Cu) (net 1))
 (segment (start 83.695 95.885) (end 83.68 95.9) (width 0.25) (layer B.Cu) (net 1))
 (via (at 120.015 85.815) (size 0.8) (drill 0.4) (layers F.Cu B.Cu) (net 1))
 (via (at 111.125 86.995) (size 0.8) (drill 0.4) (layers F.Cu B.Cu) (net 1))
 (segment (start 111.125 84.455) (end 110.49 85.09) (width 0.75) (layer B.Cu) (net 1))
 (segment (start 111.125 85.725) (end 110.49 85.09) (width 0.75) (layer B.Cu) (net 1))
 (segment (start 102.87 88.615) (end 102.87 85.09) (width 1.25) (layer B.Cu) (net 1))
 (segment (start 119.38 80.645) (end 119.38 80.01) (width 0.75) (layer B.Cu) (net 1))
 (segment (start 120.015 85.815) (end 118.835 86.995) (width 0.25) (layer F.Cu) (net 1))
 (segment (start 118.835 86.995) (end 111.125 86.995) (width 0.25) (layer F.Cu) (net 1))
 (via (at 118.745 88.265) (size 0.8) (drill 0.4) (layers F.Cu B.Cu) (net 1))
 (segment (start 118.2 83.91) (end 118.2 85.635) (width 0.25) (layer B.Cu) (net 1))
 (segment (start 118.2 84.455) (end 118.2 83.91) (width 0.75) (layer B.Cu) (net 1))
 (segment (start 118.2 85.635) (end 118.2 83.275) (width 0.75) (layer B.Cu) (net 1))
 (segment (start 118.2 83.275) (end 118.2 83.005) (width 0.75) (layer B.Cu) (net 1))
 (segment (start 118.2 83.005) (end 118.7 82.505) (width 0.75) (layer B.Cu) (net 1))
 (segment (start 118.7 82.505) (end 119.335 81.87) (width 0.75) (layer B.Cu) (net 1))
 (segment (start 111.125 86.36) (end 111.125 84.455) (width 0.75) (layer B.Cu) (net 1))
 (segment (start 111.125 86.995) (end 111.125 86.36) (width 0.75) (layer B.Cu) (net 1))
 (segment (start 111.125 86.36) (end 111.125 85.725) (width 0.75) (layer B.Cu) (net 1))
 (segment (start 95.885 87.63) (end 102.87 85.09) (width 1.25) (layer B.Cu) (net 1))
 (segment (start 87.665 95.85) (end 95.885 87.63) (width 1.25) (layer B.Cu) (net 1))
 (segment (start 83.68 95.85) (end 87.665 95.85) (width 1.25) (layer B.Cu) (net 1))
 (segment (start 121.19 77.025) (end 121.19 76.835) (width 1.25) (layer B.Cu) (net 1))
 (segment (start 119.38 78.835) (end 121.19 77.025) (width 1.25) (layer B.Cu) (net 1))
 (segment (start 119.38 80.01) (end 119.38 85.18) (width 1.25) (layer B.Cu) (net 1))
 (segment (start 119.38 85.18) (end 120.015 85.815) (width 1.25) (layer B.Cu) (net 1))
 (segment (start 119.38 82.55) (end 119.38 85.18) (width 0.75) (layer B.Cu) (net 1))
 (segment (start 118.745 83.185) (end 118.745 86.36) (width 1.25) (layer B.Cu) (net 1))
 (segment (start 118.745 86.36) (end 118.745 88.265) (width 1.25) (layer B.Cu) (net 1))
 (segment (start 118.835 86.995) (end 120.015 85.815) (width 0.75) (layer B.Cu) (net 1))
 (segment (start 118.745 86.995) (end 118.835 86.995) (width 0.75) (layer B.Cu) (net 1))
 (segment (start 102.87 85.09) (end 109.22 85.09) (width 1.25) (layer B.Cu) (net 1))
 (segment (start 109.22 85.09) (end 110.49 85.09) (width 1.25) (layer B.Cu) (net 1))
 (via (at 109.22 86.36) (size 0.8) (drill 0.4) (layers F.Cu B.Cu) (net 1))
 (segment (start 111.76 88.9) (end 111.125 88.265) (width 0.25) (layer F.Cu) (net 1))
 (segment (start 109.22 86.36) (end 109.22 85.09) (width 0.75) (layer B.Cu) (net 1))
 (segment (start 118.745 88.265) (end 118.745 89.535) (width 0.25) (layer F.Cu) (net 1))
 (segment (start 118.745 89.535) (end 112.395 89.535) (width 0.25) (layer F.Cu) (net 1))
 (segment (start 112.395 89.535) (end 111.76 88.9) (width 0.25) (layer F.Cu) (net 1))
 (segment (start 111.125 88.265) (end 110.49 88.265) (width 0.25) (layer F.Cu) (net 1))
 (segment (start 110.49 88.265) (end 109.22 86.995) (width 0.25) (layer F.Cu) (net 1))
 (segment (start 109.22 86.995) (end 109.22 86.36) (width 0.25) (layer F.Cu) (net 1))
 (via (at 109.855 61.595) (size 0.8) (drill 0.4) (layers F.Cu B.Cu) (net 5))
 (segment (start 109.22 62.23) (end 109.855 61.595) (width 0.25) (layer B.Cu) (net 5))
 (segment (start 109.22 72.39) (end 109.22 62.23) (width 0.25) (layer B.Cu) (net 5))
 (via (at 117.475 61.595) (size 0.8) (drill 0.4) (layers F.Cu B.Cu) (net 5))
 (segment (start 109.855 61.595) (end 117.475 61.595) (width 0.25) (layer F.Cu) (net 5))
 (via (at 99.06 67.945) (size 0.8) (drill 0.4) (layers F.Cu B.Cu) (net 5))
 (via (at 106.68 67.945) (size 0.8) (drill 0.4) (layers F.Cu B.Cu) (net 5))
 (segment (start 99.06 67.945) (end 106.68 67.945) (width 0.25) (layer F.Cu) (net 5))
 (segment (start 106.68 67.945) (end 109.22 67.945) (width 0.25) (layer B.Cu) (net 5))
 (segment (start 83.695 67.945) (end 83.68 67.96) (width 0.25) (layer B.Cu) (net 5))
 (segment (start 95.25 67.945) (end 83.695 67.945) (width 0.25) (layer B.Cu) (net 5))
 (segment (start 94.615 67.945) (end 95.25 67.945) (width 0.25) (layer B.Cu) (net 5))
 (segment (start 95.25 67.945) (end 99.06 67.945) (width 0.25) (layer B.Cu) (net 5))
 (segment (start 118.11 62.23) (end 121.285 62.23) (width 0.25) (layer B.Cu) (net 5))
 (segment (start 117.475 61.595) (end 118.11 62.23) (width 0.25) (layer B.Cu) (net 5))
 (segment (start 128.905 62.23) (end 121.285 62.23) (width 0.25) (layer B.Cu) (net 5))
 (segment (start 130.175 60.96) (end 128.905 62.23) (width 0.25) (layer B.Cu) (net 5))
 (segment (start 131.445 60.96) (end 130.175 60.96) (width 0.25) (layer B.Cu) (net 5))
 (segment (start 133.985 58.42) (end 131.445 60.96) (width 0.25) (layer B.Cu) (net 5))
 (segment (start 135.89 58.42) (end 133.985 58.42) (width 0.25) (layer B.Cu) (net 5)))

